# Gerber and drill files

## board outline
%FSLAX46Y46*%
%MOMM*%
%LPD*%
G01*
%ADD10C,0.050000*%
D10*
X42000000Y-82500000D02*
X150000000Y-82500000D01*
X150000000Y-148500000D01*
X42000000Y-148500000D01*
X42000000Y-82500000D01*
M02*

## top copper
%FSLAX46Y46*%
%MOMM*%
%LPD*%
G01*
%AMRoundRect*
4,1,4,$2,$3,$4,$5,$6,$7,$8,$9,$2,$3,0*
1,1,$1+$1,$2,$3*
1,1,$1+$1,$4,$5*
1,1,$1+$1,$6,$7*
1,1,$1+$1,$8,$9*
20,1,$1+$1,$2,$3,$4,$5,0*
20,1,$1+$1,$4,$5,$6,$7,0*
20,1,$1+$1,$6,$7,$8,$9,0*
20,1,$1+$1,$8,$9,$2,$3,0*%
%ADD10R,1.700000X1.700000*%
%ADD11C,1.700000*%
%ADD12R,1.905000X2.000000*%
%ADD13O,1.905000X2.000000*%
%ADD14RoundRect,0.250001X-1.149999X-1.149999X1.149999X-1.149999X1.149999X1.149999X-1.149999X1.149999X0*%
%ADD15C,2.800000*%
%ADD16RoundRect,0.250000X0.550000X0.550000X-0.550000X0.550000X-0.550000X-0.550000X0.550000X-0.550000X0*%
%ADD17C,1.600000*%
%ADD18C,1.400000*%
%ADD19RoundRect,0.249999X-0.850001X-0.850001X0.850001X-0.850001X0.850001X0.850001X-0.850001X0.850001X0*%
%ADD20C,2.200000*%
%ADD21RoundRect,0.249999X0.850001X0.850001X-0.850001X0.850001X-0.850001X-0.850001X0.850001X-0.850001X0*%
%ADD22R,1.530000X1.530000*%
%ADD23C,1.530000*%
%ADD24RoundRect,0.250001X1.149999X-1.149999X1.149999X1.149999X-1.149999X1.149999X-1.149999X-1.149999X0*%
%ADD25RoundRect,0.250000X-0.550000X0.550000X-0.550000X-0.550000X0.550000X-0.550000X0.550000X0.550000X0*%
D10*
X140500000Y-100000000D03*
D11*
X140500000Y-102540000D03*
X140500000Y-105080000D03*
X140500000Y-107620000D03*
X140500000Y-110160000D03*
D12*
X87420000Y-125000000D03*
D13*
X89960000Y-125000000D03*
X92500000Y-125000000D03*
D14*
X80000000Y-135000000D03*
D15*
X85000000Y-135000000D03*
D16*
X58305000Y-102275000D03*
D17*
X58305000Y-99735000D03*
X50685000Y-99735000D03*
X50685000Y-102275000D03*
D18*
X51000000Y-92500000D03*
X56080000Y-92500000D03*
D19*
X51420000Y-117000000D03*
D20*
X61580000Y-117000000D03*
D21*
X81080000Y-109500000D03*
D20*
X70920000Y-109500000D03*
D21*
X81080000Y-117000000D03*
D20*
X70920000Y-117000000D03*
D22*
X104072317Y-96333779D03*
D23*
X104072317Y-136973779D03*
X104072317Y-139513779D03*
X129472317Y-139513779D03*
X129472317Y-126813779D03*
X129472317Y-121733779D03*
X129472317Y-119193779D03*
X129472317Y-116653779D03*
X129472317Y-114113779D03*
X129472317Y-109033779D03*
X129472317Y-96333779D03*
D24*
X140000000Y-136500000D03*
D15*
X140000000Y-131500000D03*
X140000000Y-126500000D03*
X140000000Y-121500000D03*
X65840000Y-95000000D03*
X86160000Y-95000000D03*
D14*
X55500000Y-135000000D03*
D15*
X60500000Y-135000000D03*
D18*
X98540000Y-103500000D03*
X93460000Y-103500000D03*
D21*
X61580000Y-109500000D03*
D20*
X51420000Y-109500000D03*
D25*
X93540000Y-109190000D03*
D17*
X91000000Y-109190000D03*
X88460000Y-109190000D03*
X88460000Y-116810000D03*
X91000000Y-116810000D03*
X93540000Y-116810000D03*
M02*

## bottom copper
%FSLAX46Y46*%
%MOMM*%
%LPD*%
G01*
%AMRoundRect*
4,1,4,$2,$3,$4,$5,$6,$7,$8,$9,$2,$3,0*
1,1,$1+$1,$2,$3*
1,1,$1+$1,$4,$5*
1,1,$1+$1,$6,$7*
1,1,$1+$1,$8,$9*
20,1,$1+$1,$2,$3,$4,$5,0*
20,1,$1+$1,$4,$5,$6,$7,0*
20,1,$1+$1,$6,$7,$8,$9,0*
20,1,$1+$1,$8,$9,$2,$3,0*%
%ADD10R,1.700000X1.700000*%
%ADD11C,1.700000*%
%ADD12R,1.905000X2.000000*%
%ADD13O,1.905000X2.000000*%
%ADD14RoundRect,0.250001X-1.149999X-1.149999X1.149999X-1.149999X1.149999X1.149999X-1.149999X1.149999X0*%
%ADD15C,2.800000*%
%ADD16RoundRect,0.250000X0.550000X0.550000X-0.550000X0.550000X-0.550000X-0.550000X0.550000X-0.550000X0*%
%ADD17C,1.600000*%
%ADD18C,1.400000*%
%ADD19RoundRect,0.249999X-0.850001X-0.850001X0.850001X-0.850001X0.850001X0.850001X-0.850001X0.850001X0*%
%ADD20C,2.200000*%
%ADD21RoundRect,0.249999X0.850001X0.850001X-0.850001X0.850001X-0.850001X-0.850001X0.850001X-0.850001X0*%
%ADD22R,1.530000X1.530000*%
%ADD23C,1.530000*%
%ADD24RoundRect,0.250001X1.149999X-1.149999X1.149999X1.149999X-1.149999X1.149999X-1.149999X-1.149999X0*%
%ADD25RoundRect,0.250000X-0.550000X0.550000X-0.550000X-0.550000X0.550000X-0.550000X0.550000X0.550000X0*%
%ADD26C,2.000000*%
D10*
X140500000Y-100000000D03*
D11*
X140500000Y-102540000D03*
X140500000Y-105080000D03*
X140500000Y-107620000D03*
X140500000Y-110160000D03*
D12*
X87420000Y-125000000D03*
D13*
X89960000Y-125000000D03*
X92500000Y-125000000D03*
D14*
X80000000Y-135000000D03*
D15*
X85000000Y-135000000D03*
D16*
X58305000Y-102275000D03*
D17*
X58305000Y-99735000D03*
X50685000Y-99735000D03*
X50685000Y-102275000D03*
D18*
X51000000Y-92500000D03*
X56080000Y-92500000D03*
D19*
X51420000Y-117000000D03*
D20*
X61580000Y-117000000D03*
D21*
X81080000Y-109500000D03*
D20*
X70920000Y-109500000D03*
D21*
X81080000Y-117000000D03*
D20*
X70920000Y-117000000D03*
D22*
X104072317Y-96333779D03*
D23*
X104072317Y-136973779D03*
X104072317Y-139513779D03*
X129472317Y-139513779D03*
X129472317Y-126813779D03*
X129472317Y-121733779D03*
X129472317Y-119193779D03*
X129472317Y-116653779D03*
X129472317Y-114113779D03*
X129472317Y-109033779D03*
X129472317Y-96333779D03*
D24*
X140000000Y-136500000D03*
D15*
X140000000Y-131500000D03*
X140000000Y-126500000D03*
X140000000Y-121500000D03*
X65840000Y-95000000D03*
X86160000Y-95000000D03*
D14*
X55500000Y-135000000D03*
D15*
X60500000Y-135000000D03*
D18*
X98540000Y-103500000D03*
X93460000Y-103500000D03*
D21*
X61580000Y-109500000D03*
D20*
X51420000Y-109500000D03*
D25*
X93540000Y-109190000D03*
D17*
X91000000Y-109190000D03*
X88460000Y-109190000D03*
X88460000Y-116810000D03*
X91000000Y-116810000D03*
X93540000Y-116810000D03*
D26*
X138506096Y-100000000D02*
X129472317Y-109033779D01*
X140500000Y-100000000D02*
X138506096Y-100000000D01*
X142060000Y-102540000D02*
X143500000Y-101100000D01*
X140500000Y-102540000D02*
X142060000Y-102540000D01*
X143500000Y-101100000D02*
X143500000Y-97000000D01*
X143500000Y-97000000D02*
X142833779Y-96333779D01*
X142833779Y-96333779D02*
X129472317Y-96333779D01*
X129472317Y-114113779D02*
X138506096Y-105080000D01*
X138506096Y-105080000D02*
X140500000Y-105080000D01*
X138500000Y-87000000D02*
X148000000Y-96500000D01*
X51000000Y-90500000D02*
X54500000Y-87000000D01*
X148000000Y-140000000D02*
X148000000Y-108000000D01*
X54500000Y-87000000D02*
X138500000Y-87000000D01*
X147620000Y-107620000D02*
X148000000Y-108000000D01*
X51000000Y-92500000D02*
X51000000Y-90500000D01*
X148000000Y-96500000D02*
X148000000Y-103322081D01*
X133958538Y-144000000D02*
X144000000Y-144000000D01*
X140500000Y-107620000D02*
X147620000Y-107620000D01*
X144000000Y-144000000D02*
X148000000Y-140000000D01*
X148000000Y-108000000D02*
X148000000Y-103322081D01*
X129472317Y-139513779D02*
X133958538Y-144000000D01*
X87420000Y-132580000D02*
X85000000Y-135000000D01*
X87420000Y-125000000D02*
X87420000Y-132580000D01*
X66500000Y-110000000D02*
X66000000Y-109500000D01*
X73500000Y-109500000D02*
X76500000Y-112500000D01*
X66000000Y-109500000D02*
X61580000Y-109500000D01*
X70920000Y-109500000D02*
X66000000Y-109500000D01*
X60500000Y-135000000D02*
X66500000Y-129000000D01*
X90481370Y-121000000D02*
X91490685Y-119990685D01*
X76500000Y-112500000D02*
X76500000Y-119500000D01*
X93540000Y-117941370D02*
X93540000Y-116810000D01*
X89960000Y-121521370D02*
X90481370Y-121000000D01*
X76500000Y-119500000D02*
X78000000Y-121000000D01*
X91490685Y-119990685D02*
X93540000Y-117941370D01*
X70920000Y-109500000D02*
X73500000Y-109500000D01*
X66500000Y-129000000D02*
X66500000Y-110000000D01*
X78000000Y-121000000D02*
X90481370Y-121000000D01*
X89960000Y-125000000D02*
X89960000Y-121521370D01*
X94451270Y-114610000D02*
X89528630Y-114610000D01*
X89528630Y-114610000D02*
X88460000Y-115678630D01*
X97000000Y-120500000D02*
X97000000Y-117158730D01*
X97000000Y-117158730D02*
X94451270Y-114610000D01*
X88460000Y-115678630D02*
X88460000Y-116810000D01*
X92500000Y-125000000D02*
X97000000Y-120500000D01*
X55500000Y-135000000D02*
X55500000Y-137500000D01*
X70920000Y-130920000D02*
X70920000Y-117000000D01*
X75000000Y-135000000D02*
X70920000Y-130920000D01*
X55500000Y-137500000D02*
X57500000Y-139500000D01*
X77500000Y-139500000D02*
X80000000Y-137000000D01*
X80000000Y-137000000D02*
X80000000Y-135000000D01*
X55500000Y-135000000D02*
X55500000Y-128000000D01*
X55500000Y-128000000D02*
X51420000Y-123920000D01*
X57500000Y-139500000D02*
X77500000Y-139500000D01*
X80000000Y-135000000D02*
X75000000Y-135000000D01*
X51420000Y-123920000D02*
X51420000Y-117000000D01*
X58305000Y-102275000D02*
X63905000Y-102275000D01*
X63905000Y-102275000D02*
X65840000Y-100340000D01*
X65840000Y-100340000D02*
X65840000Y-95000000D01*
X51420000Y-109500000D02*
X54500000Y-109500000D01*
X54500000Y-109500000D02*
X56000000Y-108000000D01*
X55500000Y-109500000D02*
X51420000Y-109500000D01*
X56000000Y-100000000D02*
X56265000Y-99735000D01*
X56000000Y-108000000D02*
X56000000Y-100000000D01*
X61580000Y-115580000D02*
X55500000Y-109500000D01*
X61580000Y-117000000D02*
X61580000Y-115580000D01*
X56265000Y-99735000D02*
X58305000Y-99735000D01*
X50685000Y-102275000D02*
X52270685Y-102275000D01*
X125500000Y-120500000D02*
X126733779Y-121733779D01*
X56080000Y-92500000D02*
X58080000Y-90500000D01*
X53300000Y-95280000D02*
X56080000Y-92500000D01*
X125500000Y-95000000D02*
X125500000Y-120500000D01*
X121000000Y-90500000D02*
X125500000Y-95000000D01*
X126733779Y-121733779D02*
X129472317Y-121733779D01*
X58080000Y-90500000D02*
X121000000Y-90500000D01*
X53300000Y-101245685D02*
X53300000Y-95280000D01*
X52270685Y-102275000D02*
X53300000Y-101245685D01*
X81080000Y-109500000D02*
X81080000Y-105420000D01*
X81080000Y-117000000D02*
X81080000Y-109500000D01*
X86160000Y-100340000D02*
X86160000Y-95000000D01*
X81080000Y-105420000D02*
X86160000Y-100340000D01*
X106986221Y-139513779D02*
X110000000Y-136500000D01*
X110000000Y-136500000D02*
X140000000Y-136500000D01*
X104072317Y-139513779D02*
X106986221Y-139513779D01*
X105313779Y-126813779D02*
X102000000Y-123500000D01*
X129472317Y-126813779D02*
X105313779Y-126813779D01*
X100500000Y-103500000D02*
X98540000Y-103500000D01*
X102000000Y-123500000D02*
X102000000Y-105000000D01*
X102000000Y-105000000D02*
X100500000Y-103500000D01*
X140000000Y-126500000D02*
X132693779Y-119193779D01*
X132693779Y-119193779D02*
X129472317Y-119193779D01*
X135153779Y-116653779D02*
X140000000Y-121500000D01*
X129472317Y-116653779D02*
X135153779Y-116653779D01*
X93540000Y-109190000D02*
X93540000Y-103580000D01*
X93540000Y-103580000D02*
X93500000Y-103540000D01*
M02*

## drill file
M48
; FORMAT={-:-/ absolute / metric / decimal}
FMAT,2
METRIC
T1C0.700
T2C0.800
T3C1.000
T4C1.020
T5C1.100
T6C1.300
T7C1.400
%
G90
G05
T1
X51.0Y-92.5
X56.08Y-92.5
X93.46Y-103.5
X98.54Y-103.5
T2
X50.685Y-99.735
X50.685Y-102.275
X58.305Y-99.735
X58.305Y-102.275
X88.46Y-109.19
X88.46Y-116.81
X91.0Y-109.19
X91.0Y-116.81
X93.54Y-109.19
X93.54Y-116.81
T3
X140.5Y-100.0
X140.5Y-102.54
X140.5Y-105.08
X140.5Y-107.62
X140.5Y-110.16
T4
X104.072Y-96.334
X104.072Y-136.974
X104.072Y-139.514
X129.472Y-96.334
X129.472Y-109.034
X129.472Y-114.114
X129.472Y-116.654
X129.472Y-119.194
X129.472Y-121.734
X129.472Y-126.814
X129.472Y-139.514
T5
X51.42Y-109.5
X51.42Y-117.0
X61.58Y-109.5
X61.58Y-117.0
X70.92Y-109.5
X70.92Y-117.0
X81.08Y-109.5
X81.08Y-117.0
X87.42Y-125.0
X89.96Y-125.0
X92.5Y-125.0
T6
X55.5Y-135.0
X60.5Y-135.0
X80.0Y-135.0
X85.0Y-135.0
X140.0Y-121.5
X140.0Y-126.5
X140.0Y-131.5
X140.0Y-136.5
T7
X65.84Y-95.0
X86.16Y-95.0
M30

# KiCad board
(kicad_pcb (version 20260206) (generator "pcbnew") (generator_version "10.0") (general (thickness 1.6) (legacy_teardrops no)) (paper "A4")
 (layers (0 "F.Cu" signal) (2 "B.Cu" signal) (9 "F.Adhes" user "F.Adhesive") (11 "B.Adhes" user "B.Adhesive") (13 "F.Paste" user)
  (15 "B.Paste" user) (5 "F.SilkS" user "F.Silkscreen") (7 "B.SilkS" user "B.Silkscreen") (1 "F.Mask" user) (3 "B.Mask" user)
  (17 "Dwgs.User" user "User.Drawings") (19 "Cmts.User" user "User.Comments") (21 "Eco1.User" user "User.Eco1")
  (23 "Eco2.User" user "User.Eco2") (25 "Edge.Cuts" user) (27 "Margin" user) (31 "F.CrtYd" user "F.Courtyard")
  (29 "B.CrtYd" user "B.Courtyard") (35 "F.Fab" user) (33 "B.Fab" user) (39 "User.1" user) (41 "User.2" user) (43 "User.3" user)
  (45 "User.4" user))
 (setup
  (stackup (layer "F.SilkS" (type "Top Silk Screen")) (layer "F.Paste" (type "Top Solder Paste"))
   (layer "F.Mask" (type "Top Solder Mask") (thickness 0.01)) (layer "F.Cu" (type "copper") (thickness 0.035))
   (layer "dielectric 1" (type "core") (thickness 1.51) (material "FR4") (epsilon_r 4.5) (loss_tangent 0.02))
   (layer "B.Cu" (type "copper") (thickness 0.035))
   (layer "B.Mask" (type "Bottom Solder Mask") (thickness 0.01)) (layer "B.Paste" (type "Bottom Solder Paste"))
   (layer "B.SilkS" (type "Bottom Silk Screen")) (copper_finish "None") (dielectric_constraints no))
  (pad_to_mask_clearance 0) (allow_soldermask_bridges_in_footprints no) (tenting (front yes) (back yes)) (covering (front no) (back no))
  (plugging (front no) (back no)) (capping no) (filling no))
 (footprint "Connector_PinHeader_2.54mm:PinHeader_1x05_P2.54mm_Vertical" (layer "F.Cu") (at 140.5 100)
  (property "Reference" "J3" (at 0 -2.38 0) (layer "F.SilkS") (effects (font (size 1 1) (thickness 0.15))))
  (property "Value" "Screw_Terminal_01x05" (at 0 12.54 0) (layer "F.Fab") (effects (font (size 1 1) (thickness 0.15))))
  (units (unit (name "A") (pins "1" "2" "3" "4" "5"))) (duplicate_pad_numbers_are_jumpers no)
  (pad "1" thru_hole rect (at 0 0) (size 1.7 1.7) (drill 1) (layers "*.Cu" "*.Mask") (remove_unused_layers no) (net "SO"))
  (pad "2" thru_hole circle (at 0 2.54) (size 1.7 1.7) (drill 1) (layers "*.Cu" "*.Mask") (remove_unused_layers no) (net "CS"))
  (pad "3" thru_hole circle (at 0 5.08) (size 1.7 1.7) (drill 1) (layers "*.Cu" "*.Mask") (remove_unused_layers no) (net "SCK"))
  (pad "4" thru_hole circle (at 0 7.62) (size 1.7 1.7) (drill 1) (layers "*.Cu" "*.Mask") (remove_unused_layers no) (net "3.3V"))
  (pad "5" thru_hole circle (at 0 10.16) (size 1.7 1.7) (drill 1) (layers "*.Cu" "*.Mask") (remove_unused_layers no) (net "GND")))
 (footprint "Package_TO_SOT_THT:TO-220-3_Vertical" (layer "F.Cu") (at 87.42 125)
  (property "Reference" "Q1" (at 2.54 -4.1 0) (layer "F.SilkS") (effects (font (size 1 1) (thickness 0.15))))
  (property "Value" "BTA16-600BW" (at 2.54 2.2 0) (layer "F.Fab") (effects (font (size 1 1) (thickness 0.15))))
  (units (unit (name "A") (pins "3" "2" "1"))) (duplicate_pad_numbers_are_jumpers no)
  (pad "1" thru_hole rect (at 0 0) (size 1.905 2) (drill 1.1) (layers "*.Cu" "*.Mask") (remove_unused_layers no) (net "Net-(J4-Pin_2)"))
  (pad "2" thru_hole oval (at 2.54 0) (size 1.905 2) (drill 1.1) (layers "*.Cu" "*.Mask") (remove_unused_layers no) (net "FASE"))
  (pad "3" thru_hole oval (at 5.08 0) (size 1.905 2) (drill 1.1) (layers "*.Cu" "*.Mask") (remove_unused_layers no) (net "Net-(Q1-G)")))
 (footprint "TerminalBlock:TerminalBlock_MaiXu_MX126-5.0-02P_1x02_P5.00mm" (layer "F.Cu") (at 80 135)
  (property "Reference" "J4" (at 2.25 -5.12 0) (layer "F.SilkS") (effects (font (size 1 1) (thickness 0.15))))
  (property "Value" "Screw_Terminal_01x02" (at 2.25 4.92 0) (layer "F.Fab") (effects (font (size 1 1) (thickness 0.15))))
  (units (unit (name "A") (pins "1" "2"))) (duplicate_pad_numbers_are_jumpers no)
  (pad "1" thru_hole roundrect (at 0 0) (size 2.8 2.8) (drill 1.3) (layers "*.Cu" "*.Mask") (remove_unused_layers no)
   (roundrect_rratio 0.089286) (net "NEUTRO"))
  (pad "2" thru_hole circle (at 5 0) (size 2.8 2.8) (drill 1.3) (layers "*.Cu" "*.Mask") (remove_unused_layers no) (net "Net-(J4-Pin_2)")))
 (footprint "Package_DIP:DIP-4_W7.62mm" (layer "F.Cu") (at 58.305 102.275 180)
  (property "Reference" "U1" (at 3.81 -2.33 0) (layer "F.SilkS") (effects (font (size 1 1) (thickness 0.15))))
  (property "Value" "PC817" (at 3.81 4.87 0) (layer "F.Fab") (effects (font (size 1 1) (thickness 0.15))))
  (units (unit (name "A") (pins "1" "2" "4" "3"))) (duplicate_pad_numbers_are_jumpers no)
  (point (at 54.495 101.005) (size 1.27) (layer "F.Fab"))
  (pad "1" thru_hole roundrect (at 0 0 180) (size 1.6 1.6) (drill 0.8) (layers "*.Cu" "*.Mask") (remove_unused_layers no)
   (roundrect_rratio 0.15625) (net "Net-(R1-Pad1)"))
  (pad "2" thru_hole circle (at 0 2.54 180) (size 1.6 1.6) (drill 0.8) (layers "*.Cu" "*.Mask") (remove_unused_layers no) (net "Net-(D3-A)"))
  (pad "3" thru_hole circle (at 7.62 2.54 180) (size 1.6 1.6) (drill 0.8) (layers "*.Cu" "*.Mask") (remove_unused_layers no) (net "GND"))
  (pad "4" thru_hole circle (at 7.62 0 180) (size 1.6 1.6) (drill 0.8) (layers "*.Cu" "*.Mask") (remove_unused_layers no) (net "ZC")))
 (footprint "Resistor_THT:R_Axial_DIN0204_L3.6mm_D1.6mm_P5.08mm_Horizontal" (layer "F.Cu") (at 51 92.5)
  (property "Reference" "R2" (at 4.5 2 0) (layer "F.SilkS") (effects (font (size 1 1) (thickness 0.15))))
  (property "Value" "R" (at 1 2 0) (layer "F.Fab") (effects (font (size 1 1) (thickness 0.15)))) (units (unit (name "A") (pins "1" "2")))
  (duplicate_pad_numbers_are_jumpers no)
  (pad "1" thru_hole circle (at 0 0) (size 1.4 1.4) (drill 0.7) (layers "*.Cu" "*.Mask") (remove_unused_layers no) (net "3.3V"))
  (pad "2" thru_hole circle (at 5.08 0) (size 1.4 1.4) (drill 0.7) (layers "*.Cu" "*.Mask") (remove_unused_layers no) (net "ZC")))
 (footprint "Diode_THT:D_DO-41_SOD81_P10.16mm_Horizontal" (layer "F.Cu") (at 51.42 117)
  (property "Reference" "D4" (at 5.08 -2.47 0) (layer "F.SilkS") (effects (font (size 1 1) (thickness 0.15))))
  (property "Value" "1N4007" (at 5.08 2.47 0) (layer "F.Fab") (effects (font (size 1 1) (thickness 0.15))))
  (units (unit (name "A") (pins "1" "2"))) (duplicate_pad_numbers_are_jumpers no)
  (pad "1" thru_hole roundrect (at 0 0) (size 2.2 2.2) (drill 1.1) (layers "*.Cu" "*.Mask") (remove_unused_layers no)
   (roundrect_rratio 0.113636) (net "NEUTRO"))
  (pad "2" thru_hole circle (at 10.16 0) (size 2.2 2.2) (drill 1.1) (layers "*.Cu" "*.Mask") (remove_unused_layers no) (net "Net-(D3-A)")))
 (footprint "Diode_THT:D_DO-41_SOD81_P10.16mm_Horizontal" (layer "F.Cu") (at 81.08 109.5 180)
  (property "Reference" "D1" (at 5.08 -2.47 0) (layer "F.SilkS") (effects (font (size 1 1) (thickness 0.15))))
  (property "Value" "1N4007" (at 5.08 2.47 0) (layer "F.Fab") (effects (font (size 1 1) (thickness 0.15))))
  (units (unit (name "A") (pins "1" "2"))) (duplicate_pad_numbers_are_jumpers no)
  (pad "1" thru_hole roundrect (at 0 0 180) (size 2.2 2.2) (drill 1.1) (layers "*.Cu" "*.Mask") (remove_unused_layers no)
   (roundrect_rratio 0.113636) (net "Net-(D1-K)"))
  (pad "2" thru_hole circle (at 10.16 0 180) (size 2.2 2.2) (drill 1.1) (layers "*.Cu" "*.Mask") (remove_unused_layers no) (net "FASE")))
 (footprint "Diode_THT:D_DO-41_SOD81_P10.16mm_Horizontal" (layer "F.Cu") (at 81.08 117 180)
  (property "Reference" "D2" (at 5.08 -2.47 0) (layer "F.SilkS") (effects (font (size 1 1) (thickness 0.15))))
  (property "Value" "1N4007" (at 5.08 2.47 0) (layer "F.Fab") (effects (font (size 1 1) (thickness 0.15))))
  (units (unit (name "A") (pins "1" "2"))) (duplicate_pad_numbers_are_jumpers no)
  (pad "1" thru_hole roundrect (at 0 0 180) (size 2.2 2.2) (drill 1.1) (layers "*.Cu" "*.Mask") (remove_unused_layers no)
   (roundrect_rratio 0.113636) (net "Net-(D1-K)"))
  (pad "2" thru_hole circle (at 10.16 0 180) (size 2.2 2.2) (drill 1.1) (layers "*.Cu" "*.Mask") (remove_unused_layers no) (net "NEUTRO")))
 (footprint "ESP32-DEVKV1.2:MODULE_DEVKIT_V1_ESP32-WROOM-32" (layer "F.Cu") (at 116.772317 119.183779)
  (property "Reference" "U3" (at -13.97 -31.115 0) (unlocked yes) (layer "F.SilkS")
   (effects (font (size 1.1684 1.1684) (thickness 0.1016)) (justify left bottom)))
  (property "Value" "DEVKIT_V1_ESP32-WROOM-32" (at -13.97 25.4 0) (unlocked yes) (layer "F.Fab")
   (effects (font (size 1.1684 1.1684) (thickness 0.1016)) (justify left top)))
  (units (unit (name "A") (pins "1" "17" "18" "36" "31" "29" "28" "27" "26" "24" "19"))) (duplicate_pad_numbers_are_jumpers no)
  (pad "1" thru_hole rect (at -12.7 -22.85) (size 1.53 1.53) (drill 1.02) (layers "*.Cu" "*.Mask") (remove_unused_layers no)
   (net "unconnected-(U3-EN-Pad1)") (solder_mask_margin 0.1016) (thermal_bridge_angle 0))
  (pad "17" thru_hole circle (at -12.7 17.79) (size 1.53 1.53) (drill 1.02) (layers "*.Cu" "*.Mask") (remove_unused_layers no) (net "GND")
   (solder_mask_margin 0.1016) (thermal_bridge_angle 0))
  (pad "18" thru_hole circle (at -12.7 20.33) (size 1.53 1.53) (drill 1.02) (layers "*.Cu" "*.Mask") (remove_unused_layers no) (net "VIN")
   (solder_mask_margin 0.1016) (thermal_bridge_angle 0))
  (pad "19" thru_hole circle (at 12.7 20.33) (size 1.53 1.53) (drill 1.02) (layers "*.Cu" "*.Mask") (remove_unused_layers no) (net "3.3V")
   (solder_mask_margin 0.1016) (thermal_bridge_angle 0))
  (pad "24" thru_hole circle (at 12.7 7.63) (size 1.53 1.53) (drill 1.02) (layers "*.Cu" "*.Mask") (remove_unused_layers no) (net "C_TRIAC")
   (solder_mask_margin 0.1016) (thermal_bridge_angle 0))
  (pad "26" thru_hole circle (at 12.7 2.55) (size 1.53 1.53) (drill 1.02) (layers "*.Cu" "*.Mask") (remove_unused_layers no) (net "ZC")
   (solder_mask_margin 0.1016) (thermal_bridge_angle 0))
  (pad "27" thru_hole circle (at 12.7 0.01) (size 1.53 1.53) (drill 1.02) (layers "*.Cu" "*.Mask") (remove_unused_layers no) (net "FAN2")
   (solder_mask_margin 0.1016) (thermal_bridge_angle 0))
  (pad "28" thru_hole circle (at 12.7 -2.53) (size 1.53 1.53) (drill 1.02) (layers "*.Cu" "*.Mask") (remove_unused_layers no) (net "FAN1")
   (solder_mask_margin 0.1016) (thermal_bridge_angle 0))
  (pad "29" thru_hole circle (at 12.7 -5.07) (size 1.53 1.53) (drill 1.02) (layers "*.Cu" "*.Mask") (remove_unused_layers no) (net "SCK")
   (solder_mask_margin 0.1016) (thermal_bridge_angle 0))
  (pad "31" thru_hole circle (at 12.7 -10.15) (size 1.53 1.53) (drill 1.02) (layers "*.Cu" "*.Mask") (remove_unused_layers no) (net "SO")
   (solder_mask_margin 0.1016) (thermal_bridge_angle 0))
  (pad "36" thru_hole circle (at 12.7 -22.85) (size 1.53 1.53) (drill 1.02) (layers "*.Cu" "*.Mask") (remove_unused_layers no) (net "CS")
   (solder_mask_margin 0.1016) (thermal_bridge_angle 0)))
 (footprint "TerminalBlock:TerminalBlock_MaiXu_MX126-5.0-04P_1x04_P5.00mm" (layer "F.Cu") (at 140 136.5 90)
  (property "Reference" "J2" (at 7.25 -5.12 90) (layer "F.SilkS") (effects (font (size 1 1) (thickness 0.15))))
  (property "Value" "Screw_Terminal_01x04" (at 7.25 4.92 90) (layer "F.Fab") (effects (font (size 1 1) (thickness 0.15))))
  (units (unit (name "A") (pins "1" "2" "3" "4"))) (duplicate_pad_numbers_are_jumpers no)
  (pad "1" thru_hole roundrect (at 0 0 90) (size 2.8 2.8) (drill 1.3) (layers "*.Cu" "*.Mask") (remove_unused_layers no)
   (roundrect_rratio 0.089286) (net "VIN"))
  (pad "2" thru_hole circle (at 5 0 90) (size 2.8 2.8) (drill 1.3) (layers "*.Cu" "*.Mask") (remove_unused_layers no) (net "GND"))
  (pad "3" thru_hole circle (at 10 0 90) (size 2.8 2.8) (drill 1.3) (layers "*.Cu" "*.Mask") (remove_unused_layers no) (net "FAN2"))
  (pad "4" thru_hole circle (at 15 0 90) (size 2.8 2.8) (drill 1.3) (layers "*.Cu" "*.Mask") (remove_unused_layers no) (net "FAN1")))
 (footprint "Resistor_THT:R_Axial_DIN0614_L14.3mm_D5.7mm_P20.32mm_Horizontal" (layer "F.Cu") (at 65.84 95)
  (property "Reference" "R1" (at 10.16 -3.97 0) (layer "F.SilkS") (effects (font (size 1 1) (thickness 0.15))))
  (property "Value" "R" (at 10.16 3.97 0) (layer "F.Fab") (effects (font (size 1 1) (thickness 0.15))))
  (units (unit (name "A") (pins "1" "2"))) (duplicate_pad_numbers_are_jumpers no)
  (pad "1" thru_hole circle (at 0 0) (size 2.8 2.8) (drill 1.4) (layers "*.Cu" "*.Mask") (remove_unused_layers no) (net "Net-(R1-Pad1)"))
  (pad "2" thru_hole circle (at 20.32 0) (size 2.8 2.8) (drill 1.4) (layers "*.Cu" "*.Mask") (remove_unused_layers no) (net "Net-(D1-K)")))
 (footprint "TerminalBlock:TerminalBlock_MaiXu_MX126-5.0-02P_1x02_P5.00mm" (layer "F.Cu") (at 55.5 135)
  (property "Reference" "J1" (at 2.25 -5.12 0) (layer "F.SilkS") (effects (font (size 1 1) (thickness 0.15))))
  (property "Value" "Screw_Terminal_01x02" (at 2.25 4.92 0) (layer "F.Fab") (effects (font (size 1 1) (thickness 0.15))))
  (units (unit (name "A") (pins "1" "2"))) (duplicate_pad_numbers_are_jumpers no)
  (pad "1" thru_hole roundrect (at 0 0) (size 2.8 2.8) (drill 1.3) (layers "*.Cu" "*.Mask") (remove_unused_layers no)
   (roundrect_rratio 0.089286) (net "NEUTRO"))
  (pad "2" thru_hole circle (at 5 0) (size 2.8 2.8) (drill 1.3) (layers "*.Cu" "*.Mask") (remove_unused_layers no) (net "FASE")))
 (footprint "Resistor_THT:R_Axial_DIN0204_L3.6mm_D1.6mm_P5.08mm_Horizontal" (layer "F.Cu") (at 98.54 103.5 180)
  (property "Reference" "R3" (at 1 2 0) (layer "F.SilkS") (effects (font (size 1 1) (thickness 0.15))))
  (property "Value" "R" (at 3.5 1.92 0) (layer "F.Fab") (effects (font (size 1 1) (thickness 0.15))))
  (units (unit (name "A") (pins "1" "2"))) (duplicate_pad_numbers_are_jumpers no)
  (pad "1" thru_hole circle (at 0 0 180) (size 1.4 1.4) (drill 0.7) (layers "*.Cu" "*.Mask") (remove_unused_layers no) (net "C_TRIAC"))
  (pad "2" thru_hole circle (at 5.08 0 180) (size 1.4 1.4) (drill 0.7) (layers "*.Cu" "*.Mask") (remove_unused_layers no)
   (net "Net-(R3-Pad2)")))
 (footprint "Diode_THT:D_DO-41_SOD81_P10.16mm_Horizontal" (layer "F.Cu") (at 61.58 109.5 180)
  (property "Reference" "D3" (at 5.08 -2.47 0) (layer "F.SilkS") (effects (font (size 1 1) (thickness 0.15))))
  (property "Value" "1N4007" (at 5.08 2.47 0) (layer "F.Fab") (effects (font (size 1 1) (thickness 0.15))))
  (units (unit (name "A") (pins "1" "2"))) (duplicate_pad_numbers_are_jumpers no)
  (pad "1" thru_hole roundrect (at 0 0 180) (size 2.2 2.2) (drill 1.1) (layers "*.Cu" "*.Mask") (remove_unused_layers no)
   (roundrect_rratio 0.113636) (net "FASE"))
  (pad "2" thru_hole circle (at 10.16 0 180) (size 2.2 2.2) (drill 1.1) (layers "*.Cu" "*.Mask") (remove_unused_layers no)
   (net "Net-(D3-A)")))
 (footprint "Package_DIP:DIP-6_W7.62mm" (layer "F.Cu") (at 93.54 109.19 -90)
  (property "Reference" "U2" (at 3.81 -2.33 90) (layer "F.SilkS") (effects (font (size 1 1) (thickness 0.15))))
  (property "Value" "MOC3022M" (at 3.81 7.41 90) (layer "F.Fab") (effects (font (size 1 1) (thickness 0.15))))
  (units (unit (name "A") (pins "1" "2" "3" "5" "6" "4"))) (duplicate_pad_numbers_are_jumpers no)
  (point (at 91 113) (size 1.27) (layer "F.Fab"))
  (pad "1" thru_hole roundrect (at 0 0 270) (size 1.6 1.6) (drill 0.8) (layers "*.Cu" "*.Mask") (remove_unused_layers no)
   (roundrect_rratio 0.15625) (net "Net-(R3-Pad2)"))
  (pad "2" thru_hole circle (at 0 2.54 270) (size 1.6 1.6) (drill 0.8) (layers "*.Cu" "*.Mask") (remove_unused_layers no) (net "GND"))
  (pad "3" thru_hole circle (at 0 5.08 270) (size 1.6 1.6) (drill 0.8) (layers "*.Cu" "*.Mask") (remove_unused_layers no)
   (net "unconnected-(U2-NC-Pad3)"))
  (pad "4" thru_hole circle (at 7.62 5.08 270) (size 1.6 1.6) (drill 0.8) (layers "*.Cu" "*.Mask") (remove_unused_layers no)
   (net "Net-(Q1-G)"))
  (pad "5" thru_hole circle (at 7.62 2.54 270) (size 1.6 1.6) (drill 0.8) (layers "*.Cu" "*.Mask") (remove_unused_layers no)
   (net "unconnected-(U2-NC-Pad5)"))
  (pad "6" thru_hole circle (at 7.62 0 270) (size 1.6 1.6) (drill 0.8) (layers "*.Cu" "*.Mask") (remove_unused_layers no) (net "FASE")))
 (gr_rect (start 42 82.5) (end 150 148.5) (stroke (width 0.05) (type default)) (fill no) (layer "Edge.Cuts"))
 (segment (start 138.506096 100) (end 129.472317 109.033779) (width 2) (layer "B.Cu") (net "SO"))
 (segment (start 140.5 100) (end 138.506096 100) (width 2) (layer "B.Cu") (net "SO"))
 (segment (start 142.06 102.54) (end 143.5 101.1) (width 2) (layer "B.Cu") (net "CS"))
 (segment (start 140.5 102.54) (end 142.06 102.54) (width 2) (layer "B.Cu") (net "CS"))
 (segment (start 143.5 101.1) (end 143.5 97) (width 2) (layer "B.Cu") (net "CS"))
 (segment (start 143.5 97) (end 142.833779 96.333779) (width 2) (layer "B.Cu") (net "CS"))
 (segment (start 142.833779 96.333779) (end 129.472317 96.333779) (width 2) (layer "B.Cu") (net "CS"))
 (segment (start 129.472317 114.113779) (end 138.506096 105.08) (width 2) (layer "B.Cu") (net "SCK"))
 (segment (start 138.506096 105.08) (end 140.5 105.08) (width 2) (layer "B.Cu") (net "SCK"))
 (segment (start 138.5 87) (end 148 96.5) (width 2) (layer "B.Cu") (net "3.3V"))
 (segment (start 51 90.5) (end 54.5 87) (width 2) (layer "B.Cu") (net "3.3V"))
 (segment (start 148 140) (end 148 108) (width 2) (layer "B.Cu") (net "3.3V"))
 (segment (start 54.5 87) (end 138.5 87) (width 2) (layer "B.Cu") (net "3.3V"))
 (segment (start 147.62 107.62) (end 148 108) (width 2) (layer "B.Cu") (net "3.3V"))
 (segment (start 51 92.5) (end 51 90.5) (width 2) (layer "B.Cu") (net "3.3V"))
 (segment (start 148 96.5) (end 148 103.322081) (width 2) (layer "B.Cu") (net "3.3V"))
 (segment (start 133.958538 144) (end 144 144) (width 2) (layer "B.Cu") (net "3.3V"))
 (segment (start 140.5 107.62) (end 147.62 107.62) (width 2) (layer "B.Cu") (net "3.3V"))
 (segment (start 144 144) (end 148 140) (width 2) (layer "B.Cu") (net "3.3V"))
 (segment (start 148 108) (end 148 103.322081) (width 2) (layer "B.Cu") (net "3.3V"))
 (segment (start 129.472317 139.513779) (end 133.958538 144) (width 2) (layer "B.Cu") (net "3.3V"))
 (segment (start 87.42 132.58) (end 85 135) (width 2) (layer "B.Cu") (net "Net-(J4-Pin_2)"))
 (segment (start 87.42 125) (end 87.42 132.58) (width 2) (layer "B.Cu") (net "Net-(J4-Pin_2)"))
 (segment (start 66.5 110) (end 66 109.5) (width 2) (layer "B.Cu") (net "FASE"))
 (segment (start 73.5 109.5) (end 76.5 112.5) (width 2) (layer "B.Cu") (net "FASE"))
 (segment (start 66 109.5) (end 61.58 109.5) (width 2) (layer "B.Cu") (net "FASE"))
 (segment (start 70.92 109.5) (end 66 109.5) (width 2) (layer "B.Cu") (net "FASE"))
 (segment (start 60.5 135) (end 66.5 129) (width 2) (layer "B.Cu") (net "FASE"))
 (segment (start 90.48137 121) (end 91.490685 119.990685) (width 2) (layer "B.Cu") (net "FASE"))
 (segment (start 76.5 112.5) (end 76.5 119.5) (width 2) (layer "B.Cu") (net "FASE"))
 (segment (start 93.54 117.94137) (end 93.54 116.81) (width 2) (layer "B.Cu") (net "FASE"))
 (segment (start 89.96 121.52137) (end 90.48137 121) (width 2) (layer "B.Cu") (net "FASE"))
 (segment (start 76.5 119.5) (end 78 121) (width 2) (layer "B.Cu") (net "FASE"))
 (segment (start 91.490685 119.990685) (end 93.54 117.94137) (width 2) (layer "B.Cu") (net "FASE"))
 (segment (start 70.92 109.5) (end 73.5 109.5) (width 2) (layer "B.Cu") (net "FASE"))
 (segment (start 66.5 129) (end 66.5 110) (width 2) (layer "B.Cu") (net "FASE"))
 (segment (start 78 121) (end 90.48137 121) (width 2) (layer "B.Cu") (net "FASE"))
 (segment (start 89.96 125) (end 89.96 121.52137) (width 2) (layer "B.Cu") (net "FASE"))
 (segment (start 94.45127 114.61) (end 89.52863 114.61) (width 2) (layer "B.Cu") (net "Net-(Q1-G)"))
 (segment (start 89.52863 114.61) (end 88.46 115.67863) (width 2) (layer "B.Cu") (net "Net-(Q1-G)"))
 (segment (start 97 120.5) (end 97 117.15873) (width 2) (layer "B.Cu") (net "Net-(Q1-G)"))
 (segment (start 97 117.15873) (end 94.45127 114.61) (width 2) (layer "B.Cu") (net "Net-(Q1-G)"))
 (segment (start 88.46 115.67863) (end 88.46 116.81) (width 2) (layer "B.Cu") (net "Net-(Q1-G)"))
 (segment (start 92.5 125) (end 97 120.5) (width 2) (layer "B.Cu") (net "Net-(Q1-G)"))
 (segment (start 55.5 135) (end 55.5 137.5) (width 2) (layer "B.Cu") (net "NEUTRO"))
 (segment (start 70.92 130.92) (end 70.92 117) (width 2) (layer "B.Cu") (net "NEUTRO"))
 (segment (start 75 135) (end 70.92 130.92) (width 2) (layer "B.Cu") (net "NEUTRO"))
 (segment (start 55.5 137.5) (end 57.5 139.5) (width 2) (layer "B.Cu") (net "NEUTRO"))
 (segment (start 77.5 139.5) (end 80 137) (width 2) (layer "B.Cu") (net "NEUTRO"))
 (segment (start 80 137) (end 80 135) (width 2) (layer "B.Cu") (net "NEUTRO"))
 (segment (start 55.5 135) (end 55.5 128) (width 2) (layer "B.Cu") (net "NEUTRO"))
 (segment (start 55.5 128) (end 51.42 123.92) (width 2) (layer "B.Cu") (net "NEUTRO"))
 (segment (start 57.5 139.5) (end 77.5 139.5) (width 2) (layer "B.Cu") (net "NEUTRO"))
 (segment (start 80 135) (end 75 135) (width 2) (layer "B.Cu") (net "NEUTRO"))
 (segment (start 51.42 123.92) (end 51.42 117) (width 2) (layer "B.Cu") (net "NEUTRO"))
 (segment (start 58.305 102.275) (end 63.905 102.275) (width 2) (layer "B.Cu") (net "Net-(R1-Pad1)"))
 (segment (start 63.905 102.275) (end 65.84 100.34) (width 2) (layer "B.Cu") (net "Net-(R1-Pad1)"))
 (segment (start 65.84 100.34) (end 65.84 95) (width 2) (layer "B.Cu") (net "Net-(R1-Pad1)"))
 (segment (start 51.42 109.5) (end 54.5 109.5) (width 2) (layer "B.Cu") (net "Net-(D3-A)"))
 (segment (start 54.5 109.5) (end 56 108) (width 2) (layer "B.Cu") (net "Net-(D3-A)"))
 (segment (start 55.5 109.5) (end 51.42 109.5) (width 2) (layer "B.Cu") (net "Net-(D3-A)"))
 (segment (start 56 100) (end 56.265 99.735) (width 2) (layer "B.Cu") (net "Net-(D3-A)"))
 (segment (start 56 108) (end 56 100) (width 2) (layer "B.Cu") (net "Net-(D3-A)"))
 (segment (start 61.58 115.58) (end 55.5 109.5) (width 2) (layer "B.Cu") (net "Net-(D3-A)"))
 (segment (start 61.58 117) (end 61.58 115.58) (width 2) (layer "B.Cu") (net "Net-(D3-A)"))
 (segment (start 56.265 99.735) (end 58.305 99.735) (width 2) (layer "B.Cu") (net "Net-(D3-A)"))
 (segment (start 50.685 102.275) (end 52.270685 102.275) (width 2) (layer "B.Cu") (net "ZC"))
 (segment (start 125.5 120.5) (end 126.733779 121.733779) (width 2) (layer "B.Cu") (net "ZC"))
 (segment (start 56.08 92.5) (end 58.08 90.5) (width 2) (layer "B.Cu") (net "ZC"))
 (segment (start 53.3 95.28) (end 56.08 92.5) (width 2) (layer "B.Cu") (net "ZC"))
 (segment (start 125.5 95) (end 125.5 120.5) (width 2) (layer "B.Cu") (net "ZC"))
 (segment (start 121 90.5) (end 125.5 95) (width 2) (layer "B.Cu") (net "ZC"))
 (segment (start 126.733779 121.733779) (end 129.472317 121.733779) (width 2) (layer "B.Cu") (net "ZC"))
 (segment (start 58.08 90.5) (end 121 90.5) (width 2) (layer "B.Cu") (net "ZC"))
 (segment (start 53.3 101.245685) (end 53.3 95.28) (width 2) (layer "B.Cu") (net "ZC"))
 (segment (start 52.270685 102.275) (end 53.3 101.245685) (width 2) (layer "B.Cu") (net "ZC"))
 (segment (start 81.08 109.5) (end 81.08 105.42) (width 2) (layer "B.Cu") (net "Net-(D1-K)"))
 (segment (start 81.08 117) (end 81.08 109.5) (width 2) (layer "B.Cu") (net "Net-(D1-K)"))
 (segment (start 86.16 100.34) (end 86.16 95) (width 2) (layer "B.Cu") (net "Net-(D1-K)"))
 (segment (start 81.08 105.42) (end 86.16 100.34) (width 2) (layer "B.Cu") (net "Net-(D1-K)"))
 (segment (start 106.986221 139.513779) (end 110 136.5) (width 2) (layer "B.Cu") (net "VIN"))
 (segment (start 110 136.5) (end 140 136.5) (width 2) (layer "B.Cu") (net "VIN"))
 (segment (start 104.072317 139.513779) (end 106.986221 139.513779) (width 2) (layer "B.Cu") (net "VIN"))
 (segment (start 105.313779 126.813779) (end 102 123.5) (width 2) (layer "B.Cu") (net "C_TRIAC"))
 (segment (start 129.472317 126.813779) (end 105.313779 126.813779) (width 2) (layer "B.Cu") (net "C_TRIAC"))
 (segment (start 100.5 103.5) (end 98.54 103.5) (width 2) (layer "B.Cu") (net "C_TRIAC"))
 (segment (start 102 123.5) (end 102 105) (width 2) (layer "B.Cu") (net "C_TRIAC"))
 (segment (start 102 105) (end 100.5 103.5) (width 2) (layer "B.Cu") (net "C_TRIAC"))
 (segment (start 140 126.5) (end 132.693779 119.193779) (width 2) (layer "B.Cu") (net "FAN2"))
 (segment (start 132.693779 119.193779) (end 129.472317 119.193779) (width 2) (layer "B.Cu") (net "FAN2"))
 (segment (start 135.153779 116.653779) (end 140 121.5) (width 2) (layer "B.Cu") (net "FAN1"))
 (segment (start 129.472317 116.653779) (end 135.153779 116.653779) (width 2) (layer "B.Cu") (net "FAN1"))
 (segment (start 93.54 109.19) (end 93.54 103.58) (width 2) (layer "B.Cu") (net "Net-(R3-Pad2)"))
 (segment (start 93.54 103.58) (end 93.5 103.54) (width 2) (layer "B.Cu") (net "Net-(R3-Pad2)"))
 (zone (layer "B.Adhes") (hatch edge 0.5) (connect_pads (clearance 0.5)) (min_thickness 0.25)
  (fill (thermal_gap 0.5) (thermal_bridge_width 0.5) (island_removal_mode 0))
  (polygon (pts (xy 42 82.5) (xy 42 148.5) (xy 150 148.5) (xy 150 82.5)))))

